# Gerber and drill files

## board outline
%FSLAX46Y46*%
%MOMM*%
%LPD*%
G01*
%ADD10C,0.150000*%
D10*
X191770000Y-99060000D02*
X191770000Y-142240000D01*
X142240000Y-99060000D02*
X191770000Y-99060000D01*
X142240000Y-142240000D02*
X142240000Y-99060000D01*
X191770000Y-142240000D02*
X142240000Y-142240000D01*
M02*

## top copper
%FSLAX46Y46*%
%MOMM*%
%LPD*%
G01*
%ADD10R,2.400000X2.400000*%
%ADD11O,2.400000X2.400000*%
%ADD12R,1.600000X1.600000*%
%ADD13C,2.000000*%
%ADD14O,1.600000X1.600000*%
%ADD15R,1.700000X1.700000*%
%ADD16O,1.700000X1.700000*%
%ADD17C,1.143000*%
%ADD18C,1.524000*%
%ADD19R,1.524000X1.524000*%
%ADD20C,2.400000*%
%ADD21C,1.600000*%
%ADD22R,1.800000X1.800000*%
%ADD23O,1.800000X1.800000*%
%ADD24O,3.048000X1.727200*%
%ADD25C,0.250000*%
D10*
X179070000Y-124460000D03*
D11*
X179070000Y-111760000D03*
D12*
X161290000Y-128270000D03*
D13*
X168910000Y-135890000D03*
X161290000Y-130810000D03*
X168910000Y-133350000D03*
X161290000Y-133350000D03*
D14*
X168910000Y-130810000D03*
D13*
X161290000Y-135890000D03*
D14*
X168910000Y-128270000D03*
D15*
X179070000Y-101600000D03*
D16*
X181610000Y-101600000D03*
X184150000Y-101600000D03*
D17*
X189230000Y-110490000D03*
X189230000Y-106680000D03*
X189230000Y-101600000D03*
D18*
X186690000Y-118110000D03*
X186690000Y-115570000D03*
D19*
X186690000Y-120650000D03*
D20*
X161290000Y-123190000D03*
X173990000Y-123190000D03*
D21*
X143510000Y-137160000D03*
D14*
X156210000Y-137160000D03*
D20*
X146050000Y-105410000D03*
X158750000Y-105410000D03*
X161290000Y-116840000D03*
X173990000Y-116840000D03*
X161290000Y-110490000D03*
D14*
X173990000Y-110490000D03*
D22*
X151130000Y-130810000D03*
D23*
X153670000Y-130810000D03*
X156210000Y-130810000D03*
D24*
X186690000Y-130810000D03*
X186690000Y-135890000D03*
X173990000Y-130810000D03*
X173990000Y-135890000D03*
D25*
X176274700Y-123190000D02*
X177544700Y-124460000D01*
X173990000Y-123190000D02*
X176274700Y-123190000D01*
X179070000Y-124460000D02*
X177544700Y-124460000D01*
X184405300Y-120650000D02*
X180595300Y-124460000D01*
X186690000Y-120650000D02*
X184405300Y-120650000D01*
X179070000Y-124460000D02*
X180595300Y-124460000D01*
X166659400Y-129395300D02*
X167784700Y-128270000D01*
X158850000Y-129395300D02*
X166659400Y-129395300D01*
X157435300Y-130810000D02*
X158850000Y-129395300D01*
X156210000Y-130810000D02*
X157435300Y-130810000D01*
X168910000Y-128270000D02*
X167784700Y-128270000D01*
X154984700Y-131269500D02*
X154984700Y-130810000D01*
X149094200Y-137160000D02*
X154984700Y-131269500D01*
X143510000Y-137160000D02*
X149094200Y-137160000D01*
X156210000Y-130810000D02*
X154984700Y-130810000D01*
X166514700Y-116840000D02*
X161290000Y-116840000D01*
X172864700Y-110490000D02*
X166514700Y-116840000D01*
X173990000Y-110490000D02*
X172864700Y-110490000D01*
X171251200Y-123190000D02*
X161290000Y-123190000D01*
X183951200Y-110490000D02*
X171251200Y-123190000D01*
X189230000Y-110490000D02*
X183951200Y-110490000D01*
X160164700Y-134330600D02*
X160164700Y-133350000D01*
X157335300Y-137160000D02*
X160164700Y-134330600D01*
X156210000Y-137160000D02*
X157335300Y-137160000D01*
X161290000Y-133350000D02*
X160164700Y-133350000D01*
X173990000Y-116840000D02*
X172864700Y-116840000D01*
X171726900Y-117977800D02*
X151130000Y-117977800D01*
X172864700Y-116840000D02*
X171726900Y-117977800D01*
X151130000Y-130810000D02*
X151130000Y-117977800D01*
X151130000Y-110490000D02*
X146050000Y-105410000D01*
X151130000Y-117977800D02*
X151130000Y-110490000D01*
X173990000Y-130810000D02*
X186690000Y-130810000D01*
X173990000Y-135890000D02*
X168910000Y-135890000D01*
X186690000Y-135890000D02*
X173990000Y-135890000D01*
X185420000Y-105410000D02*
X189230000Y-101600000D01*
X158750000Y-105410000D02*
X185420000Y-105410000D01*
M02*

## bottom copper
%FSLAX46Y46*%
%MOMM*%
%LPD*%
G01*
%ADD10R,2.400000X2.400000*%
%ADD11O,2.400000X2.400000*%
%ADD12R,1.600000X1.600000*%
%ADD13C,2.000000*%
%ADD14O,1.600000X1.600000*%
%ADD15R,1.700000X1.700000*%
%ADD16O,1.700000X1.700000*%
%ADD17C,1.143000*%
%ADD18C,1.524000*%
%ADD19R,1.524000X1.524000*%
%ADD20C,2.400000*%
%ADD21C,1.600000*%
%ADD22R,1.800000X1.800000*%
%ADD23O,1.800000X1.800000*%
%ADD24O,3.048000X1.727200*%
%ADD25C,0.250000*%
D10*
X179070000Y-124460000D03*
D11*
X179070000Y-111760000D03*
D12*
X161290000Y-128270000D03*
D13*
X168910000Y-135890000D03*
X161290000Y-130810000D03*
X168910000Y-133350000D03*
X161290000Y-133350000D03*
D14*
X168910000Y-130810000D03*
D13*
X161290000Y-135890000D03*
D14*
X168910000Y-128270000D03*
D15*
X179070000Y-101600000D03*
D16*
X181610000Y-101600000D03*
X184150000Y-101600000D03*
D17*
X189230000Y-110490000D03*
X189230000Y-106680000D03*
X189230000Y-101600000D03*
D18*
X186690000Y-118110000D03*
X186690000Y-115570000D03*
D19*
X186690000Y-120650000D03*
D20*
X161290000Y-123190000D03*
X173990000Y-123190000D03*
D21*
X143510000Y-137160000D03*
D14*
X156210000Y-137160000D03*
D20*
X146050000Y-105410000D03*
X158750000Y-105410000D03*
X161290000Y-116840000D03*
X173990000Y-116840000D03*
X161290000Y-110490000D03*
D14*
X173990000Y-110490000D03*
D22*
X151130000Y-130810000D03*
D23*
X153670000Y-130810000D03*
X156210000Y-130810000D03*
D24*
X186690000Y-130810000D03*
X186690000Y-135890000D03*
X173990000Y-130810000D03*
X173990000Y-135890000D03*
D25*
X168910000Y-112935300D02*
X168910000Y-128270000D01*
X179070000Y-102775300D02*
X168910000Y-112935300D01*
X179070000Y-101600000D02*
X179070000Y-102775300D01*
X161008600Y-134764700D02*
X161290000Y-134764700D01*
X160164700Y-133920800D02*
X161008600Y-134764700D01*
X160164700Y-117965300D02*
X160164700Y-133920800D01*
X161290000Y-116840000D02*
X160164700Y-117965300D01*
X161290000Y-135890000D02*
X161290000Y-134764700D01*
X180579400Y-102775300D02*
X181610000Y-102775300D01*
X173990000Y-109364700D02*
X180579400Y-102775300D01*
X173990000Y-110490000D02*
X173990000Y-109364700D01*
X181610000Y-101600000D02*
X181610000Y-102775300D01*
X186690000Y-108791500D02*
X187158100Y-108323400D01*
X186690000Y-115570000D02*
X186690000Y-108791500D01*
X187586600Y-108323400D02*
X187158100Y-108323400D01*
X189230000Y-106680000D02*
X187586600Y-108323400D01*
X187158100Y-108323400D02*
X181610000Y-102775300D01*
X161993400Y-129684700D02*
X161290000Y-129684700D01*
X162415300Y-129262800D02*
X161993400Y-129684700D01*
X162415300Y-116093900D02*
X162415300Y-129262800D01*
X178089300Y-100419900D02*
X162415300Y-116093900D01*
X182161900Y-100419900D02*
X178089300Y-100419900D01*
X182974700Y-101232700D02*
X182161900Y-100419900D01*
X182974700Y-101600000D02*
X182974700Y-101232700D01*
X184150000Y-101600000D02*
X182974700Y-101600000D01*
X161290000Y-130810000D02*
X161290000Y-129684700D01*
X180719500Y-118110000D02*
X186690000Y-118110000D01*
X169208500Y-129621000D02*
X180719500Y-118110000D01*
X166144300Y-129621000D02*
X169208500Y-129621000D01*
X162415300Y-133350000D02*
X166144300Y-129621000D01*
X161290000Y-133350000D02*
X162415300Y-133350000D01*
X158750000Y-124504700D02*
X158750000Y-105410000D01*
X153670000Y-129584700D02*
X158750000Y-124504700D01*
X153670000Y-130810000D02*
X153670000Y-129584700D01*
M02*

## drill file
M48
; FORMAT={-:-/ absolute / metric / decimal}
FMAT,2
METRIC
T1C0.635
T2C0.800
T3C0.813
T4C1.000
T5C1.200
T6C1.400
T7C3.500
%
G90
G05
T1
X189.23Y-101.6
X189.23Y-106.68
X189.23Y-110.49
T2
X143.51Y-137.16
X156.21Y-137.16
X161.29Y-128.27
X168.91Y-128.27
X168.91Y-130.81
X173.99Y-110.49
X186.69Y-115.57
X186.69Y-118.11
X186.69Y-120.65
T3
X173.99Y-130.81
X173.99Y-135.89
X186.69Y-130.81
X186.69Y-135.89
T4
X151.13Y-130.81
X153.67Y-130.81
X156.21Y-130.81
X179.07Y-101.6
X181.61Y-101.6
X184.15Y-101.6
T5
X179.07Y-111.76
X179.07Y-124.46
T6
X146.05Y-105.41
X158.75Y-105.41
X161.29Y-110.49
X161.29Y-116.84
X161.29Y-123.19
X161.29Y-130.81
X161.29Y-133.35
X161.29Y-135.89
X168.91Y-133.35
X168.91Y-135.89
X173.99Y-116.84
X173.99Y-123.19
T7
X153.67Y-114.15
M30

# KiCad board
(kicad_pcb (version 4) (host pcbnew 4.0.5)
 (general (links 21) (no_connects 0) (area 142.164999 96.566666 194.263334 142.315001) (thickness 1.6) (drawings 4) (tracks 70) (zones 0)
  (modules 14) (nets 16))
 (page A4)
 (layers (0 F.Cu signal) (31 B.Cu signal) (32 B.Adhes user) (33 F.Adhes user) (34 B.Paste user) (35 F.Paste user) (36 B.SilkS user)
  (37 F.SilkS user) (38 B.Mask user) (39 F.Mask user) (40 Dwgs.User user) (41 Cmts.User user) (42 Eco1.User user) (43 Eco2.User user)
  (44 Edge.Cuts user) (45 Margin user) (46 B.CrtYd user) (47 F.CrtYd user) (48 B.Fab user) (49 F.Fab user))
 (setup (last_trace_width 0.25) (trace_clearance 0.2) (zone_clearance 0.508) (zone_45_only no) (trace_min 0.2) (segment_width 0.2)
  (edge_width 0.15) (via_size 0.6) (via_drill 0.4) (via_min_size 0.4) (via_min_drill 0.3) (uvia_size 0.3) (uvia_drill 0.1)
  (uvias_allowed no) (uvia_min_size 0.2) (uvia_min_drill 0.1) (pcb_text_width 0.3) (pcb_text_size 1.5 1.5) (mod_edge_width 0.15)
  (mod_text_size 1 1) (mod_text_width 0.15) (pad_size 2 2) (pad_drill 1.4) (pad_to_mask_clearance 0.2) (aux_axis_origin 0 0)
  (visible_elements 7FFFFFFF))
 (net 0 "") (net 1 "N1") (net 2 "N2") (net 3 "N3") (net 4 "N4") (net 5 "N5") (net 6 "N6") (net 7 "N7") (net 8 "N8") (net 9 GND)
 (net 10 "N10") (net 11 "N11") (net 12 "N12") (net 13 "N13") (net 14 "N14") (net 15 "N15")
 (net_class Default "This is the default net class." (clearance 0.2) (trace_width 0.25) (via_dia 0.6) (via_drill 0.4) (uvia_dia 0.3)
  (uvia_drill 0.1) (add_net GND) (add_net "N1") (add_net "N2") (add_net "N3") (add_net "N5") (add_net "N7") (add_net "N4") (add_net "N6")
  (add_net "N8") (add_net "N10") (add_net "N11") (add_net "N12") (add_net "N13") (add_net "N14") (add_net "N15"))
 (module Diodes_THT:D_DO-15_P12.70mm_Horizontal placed (layer F.Cu) (at 179.07 124.46 90)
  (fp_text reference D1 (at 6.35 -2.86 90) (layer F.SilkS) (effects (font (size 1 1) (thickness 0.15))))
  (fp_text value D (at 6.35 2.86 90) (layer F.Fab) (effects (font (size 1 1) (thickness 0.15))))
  (pad 1 thru_hole rect (at 0 0 90) (size 2.4 2.4) (drill 1.2) (layers *.Cu *.Mask) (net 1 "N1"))
  (pad 2 thru_hole oval (at 12.7 0 90) (size 2.4 2.4) (drill 1.2) (layers *.Cu *.Mask) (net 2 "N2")))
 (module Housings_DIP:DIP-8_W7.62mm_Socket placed (layer F.Cu) (at 161.29 128.27)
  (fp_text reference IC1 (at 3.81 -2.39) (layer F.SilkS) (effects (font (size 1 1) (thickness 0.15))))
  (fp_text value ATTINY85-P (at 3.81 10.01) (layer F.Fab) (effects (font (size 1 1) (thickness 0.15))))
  (pad 1 thru_hole rect (at 0 0) (size 1.6 1.6) (drill 0.8) (layers *.Cu *.Mask) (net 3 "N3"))
  (pad 5 thru_hole circle (at 7.62 7.62) (size 2 2) (drill 1.4) (layers *.Cu *.Mask) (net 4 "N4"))
  (pad 2 thru_hole circle (at 0 2.54) (size 2 2) (drill 1.4) (layers *.Cu *.Mask) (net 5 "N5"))
  (pad 6 thru_hole circle (at 7.62 5.08) (size 2 2) (drill 1.4) (layers *.Cu *.Mask) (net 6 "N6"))
  (pad 3 thru_hole circle (at 0 5.08) (size 2 2) (drill 1.4) (layers *.Cu *.Mask) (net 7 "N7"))
  (pad 7 thru_hole oval (at 7.62 2.54) (size 1.6 1.6) (drill 0.8) (layers *.Cu *.Mask) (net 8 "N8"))
  (pad 4 thru_hole circle (at 0 7.62) (size 2 2) (drill 1.4) (layers *.Cu *.Mask) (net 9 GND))
  (pad 8 thru_hole oval (at 7.62 0) (size 1.6 1.6) (drill 0.8) (layers *.Cu *.Mask) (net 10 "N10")))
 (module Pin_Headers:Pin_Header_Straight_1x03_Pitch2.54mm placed (layer F.Cu) (at 179.07 101.6 90)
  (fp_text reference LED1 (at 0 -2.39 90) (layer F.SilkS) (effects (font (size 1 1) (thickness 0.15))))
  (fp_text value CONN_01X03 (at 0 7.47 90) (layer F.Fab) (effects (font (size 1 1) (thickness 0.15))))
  (pad 1 thru_hole rect (at 0 0 90) (size 1.7 1.7) (drill 1) (layers *.Cu *.Mask) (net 10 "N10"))
  (pad 2 thru_hole oval (at 0 2.54 90) (size 1.7 1.7) (drill 1) (layers *.Cu *.Mask) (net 9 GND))
  (pad 3 thru_hole oval (at 0 5.08 90) (size 1.7 1.7) (drill 1) (layers *.Cu *.Mask) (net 5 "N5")))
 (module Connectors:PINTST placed (layer F.Cu) (at 189.23 110.49)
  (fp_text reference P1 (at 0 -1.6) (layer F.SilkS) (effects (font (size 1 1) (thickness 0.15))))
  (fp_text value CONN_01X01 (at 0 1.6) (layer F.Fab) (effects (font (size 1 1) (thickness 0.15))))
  (pad 1 thru_hole circle (at 0 0) (size 1.143 1.143) (drill 0.635) (layers *.Cu *.Mask) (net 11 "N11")))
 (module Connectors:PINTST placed (layer F.Cu) (at 189.23 106.68)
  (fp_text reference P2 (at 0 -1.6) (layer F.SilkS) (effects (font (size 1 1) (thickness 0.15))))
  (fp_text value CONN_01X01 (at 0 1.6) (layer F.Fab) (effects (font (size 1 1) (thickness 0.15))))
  (pad 1 thru_hole circle (at 0 0) (size 1.143 1.143) (drill 0.635) (layers *.Cu *.Mask) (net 9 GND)))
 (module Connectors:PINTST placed (layer F.Cu) (at 189.23 101.6)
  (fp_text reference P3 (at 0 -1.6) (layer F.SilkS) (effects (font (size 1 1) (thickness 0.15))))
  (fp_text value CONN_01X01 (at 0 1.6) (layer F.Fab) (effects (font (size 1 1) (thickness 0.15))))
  (pad 1 thru_hole circle (at 0 0) (size 1.143 1.143) (drill 0.635) (layers *.Cu *.Mask) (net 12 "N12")))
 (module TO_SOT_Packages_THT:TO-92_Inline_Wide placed (layer F.Cu) (at 186.69 120.65 90)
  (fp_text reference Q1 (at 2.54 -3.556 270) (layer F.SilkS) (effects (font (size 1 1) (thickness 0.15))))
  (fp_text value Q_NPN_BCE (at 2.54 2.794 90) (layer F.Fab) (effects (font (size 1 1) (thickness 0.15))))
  (pad 2 thru_hole circle (at 2.54 0 180) (size 1.524 1.524) (drill 0.8) (layers *.Cu *.Mask) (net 7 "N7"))
  (pad 3 thru_hole circle (at 5.08 0 180) (size 1.524 1.524) (drill 0.8) (layers *.Cu *.Mask) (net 9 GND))
  (pad 1 thru_hole rect (at 0 0 180) (size 1.524 1.524) (drill 0.8) (layers *.Cu *.Mask) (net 1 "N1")))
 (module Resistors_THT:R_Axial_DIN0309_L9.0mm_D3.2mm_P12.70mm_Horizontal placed (layer F.Cu) (at 161.29 123.19)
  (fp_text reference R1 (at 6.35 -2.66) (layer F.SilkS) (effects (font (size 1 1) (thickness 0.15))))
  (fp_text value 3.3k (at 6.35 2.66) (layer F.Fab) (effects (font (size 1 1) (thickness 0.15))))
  (pad 1 thru_hole circle (at 0 0) (size 2.4 2.4) (drill 1.4) (layers *.Cu *.Mask) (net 11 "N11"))
  (pad 2 thru_hole circle (at 12.7 0) (size 2.4 2.4) (drill 1.4) (layers *.Cu *.Mask) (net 1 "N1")))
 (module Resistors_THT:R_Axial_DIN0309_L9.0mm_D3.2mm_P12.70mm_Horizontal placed (layer F.Cu) (at 143.51 137.16)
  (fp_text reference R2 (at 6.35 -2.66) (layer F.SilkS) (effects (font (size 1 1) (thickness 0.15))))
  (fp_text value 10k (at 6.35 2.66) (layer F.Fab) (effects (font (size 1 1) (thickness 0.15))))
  (pad 1 thru_hole circle (at 0 0) (size 1.6 1.6) (drill 0.8) (layers *.Cu *.Mask) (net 10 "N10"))
  (pad 2 thru_hole oval (at 12.7 0) (size 1.6 1.6) (drill 0.8) (layers *.Cu *.Mask) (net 7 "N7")))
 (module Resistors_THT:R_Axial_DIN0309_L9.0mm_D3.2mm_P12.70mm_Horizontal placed (layer F.Cu) (at 146.05 105.41)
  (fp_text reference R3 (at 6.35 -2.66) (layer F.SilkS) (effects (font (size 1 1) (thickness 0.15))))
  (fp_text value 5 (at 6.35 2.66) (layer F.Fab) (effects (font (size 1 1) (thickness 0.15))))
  (pad 1 thru_hole circle (at 0 0) (size 2.4 2.4) (drill 1.4) (layers *.Cu *.Mask) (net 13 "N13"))
  (pad 2 thru_hole circle (at 12.7 0) (size 2.4 2.4) (drill 1.4) (layers *.Cu *.Mask) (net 12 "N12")))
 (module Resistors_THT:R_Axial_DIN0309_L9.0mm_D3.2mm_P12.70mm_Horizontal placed (layer F.Cu) (at 161.29 116.84)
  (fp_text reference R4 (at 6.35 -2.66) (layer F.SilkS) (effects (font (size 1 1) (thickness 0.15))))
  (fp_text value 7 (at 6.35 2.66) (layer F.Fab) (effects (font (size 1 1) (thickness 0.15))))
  (pad 1 thru_hole circle (at 0 0) (size 2.4 2.4) (drill 1.4) (layers *.Cu *.Mask) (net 9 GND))
  (pad 2 thru_hole circle (at 12.7 0) (size 2.4 2.4) (drill 1.4) (layers *.Cu *.Mask) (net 13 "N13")))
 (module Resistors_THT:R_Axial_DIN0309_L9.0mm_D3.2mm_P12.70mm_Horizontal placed (layer F.Cu) (at 161.29 110.49)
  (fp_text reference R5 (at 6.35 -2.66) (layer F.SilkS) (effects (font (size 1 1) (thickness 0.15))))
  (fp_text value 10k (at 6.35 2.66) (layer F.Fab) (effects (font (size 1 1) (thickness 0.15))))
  (pad 1 thru_hole circle (at 0 0) (size 2.4 2.4) (drill 1.4) (layers *.Cu *.Mask) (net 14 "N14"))
  (pad 2 thru_hole oval (at 12.7 0) (size 1.6 1.6) (drill 0.8) (layers *.Cu *.Mask) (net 9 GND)))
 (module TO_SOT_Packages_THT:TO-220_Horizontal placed (layer F.Cu) (at 151.13 130.81)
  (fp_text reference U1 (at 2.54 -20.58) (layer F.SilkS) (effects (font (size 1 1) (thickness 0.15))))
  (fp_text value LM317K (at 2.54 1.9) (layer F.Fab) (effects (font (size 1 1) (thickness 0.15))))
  (pad None np_thru_hole oval (at 2.54 -16.66) (size 3.5 3.5) (drill 3.5) (layers *.Cu *.Mask))
  (pad 1 thru_hole rect (at 0 0) (size 1.8 1.8) (drill 1) (layers *.Cu *.Mask) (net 13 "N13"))
  (pad 2 thru_hole oval (at 2.54 0) (size 1.8 1.8) (drill 1) (layers *.Cu *.Mask) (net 12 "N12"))
  (pad 3 thru_hole oval (at 5.08 0) (size 1.8 1.8) (drill 1) (layers *.Cu *.Mask) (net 10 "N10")))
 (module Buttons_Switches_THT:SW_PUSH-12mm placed (layer F.Cu) (at 180.34 133.35)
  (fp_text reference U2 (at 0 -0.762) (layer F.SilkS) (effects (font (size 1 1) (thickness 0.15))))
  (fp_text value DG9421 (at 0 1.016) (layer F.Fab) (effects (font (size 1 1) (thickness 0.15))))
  (pad 1 thru_hole oval (at 6.35 -2.54) (size 3.048 1.7272) (drill 0.8128) (layers *.Cu *.Mask) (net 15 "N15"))
  (pad 2 thru_hole oval (at 6.35 2.54) (size 3.048 1.7272) (drill 0.8128) (layers *.Cu *.Mask) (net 4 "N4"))
  (pad 1 thru_hole oval (at -6.35 -2.54) (size 3.048 1.7272) (drill 0.8128) (layers *.Cu *.Mask) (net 15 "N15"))
  (pad 2 thru_hole oval (at -6.35 2.54) (size 3.048 1.7272) (drill 0.8128) (layers *.Cu *.Mask) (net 4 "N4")))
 (gr_line (start 191.77 99.06) (end 191.77 142.24) (angle 90) (layer Edge.Cuts) (width 0.15))
 (gr_line (start 142.24 99.06) (end 191.77 99.06) (angle 90) (layer Edge.Cuts) (width 0.15))
 (gr_line (start 142.24 142.24) (end 142.24 99.06) (angle 90) (layer Edge.Cuts) (width 0.15))
 (gr_line (start 191.77 142.24) (end 142.24 142.24) (angle 90) (layer Edge.Cuts) (width 0.15))
 (segment (start 176.2747 123.19) (end 177.5447 124.46) (width 0.25) (layer F.Cu) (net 1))
 (segment (start 173.99 123.19) (end 176.2747 123.19) (width 0.25) (layer F.Cu) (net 1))
 (segment (start 179.07 124.46) (end 177.5447 124.46) (width 0.25) (layer F.Cu) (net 1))
 (segment (start 184.4053 120.65) (end 180.5953 124.46) (width 0.25) (layer F.Cu) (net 1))
 (segment (start 186.69 120.65) (end 184.4053 120.65) (width 0.25) (layer F.Cu) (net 1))
 (segment (start 179.07 124.46) (end 180.5953 124.46) (width 0.25) (layer F.Cu) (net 1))
 (segment (start 166.6594 129.3953) (end 167.7847 128.27) (width 0.25) (layer F.Cu) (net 10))
 (segment (start 158.85 129.3953) (end 166.6594 129.3953) (width 0.25) (layer F.Cu) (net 10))
 (segment (start 157.4353 130.81) (end 158.85 129.3953) (width 0.25) (layer F.Cu) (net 10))
 (segment (start 156.21 130.81) (end 157.4353 130.81) (width 0.25) (layer F.Cu) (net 10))
 (segment (start 168.91 128.27) (end 167.7847 128.27) (width 0.25) (layer F.Cu) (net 10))
 (segment (start 154.9847 131.2695) (end 154.9847 130.81) (width 0.25) (layer F.Cu) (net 10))
 (segment (start 149.0942 137.16) (end 154.9847 131.2695) (width 0.25) (layer F.Cu) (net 10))
 (segment (start 143.51 137.16) (end 149.0942 137.16) (width 0.25) (layer F.Cu) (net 10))
 (segment (start 156.21 130.81) (end 154.9847 130.81) (width 0.25) (layer F.Cu) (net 10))
 (segment (start 168.91 112.9353) (end 168.91 128.27) (width 0.25) (layer B.Cu) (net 10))
 (segment (start 179.07 102.7753) (end 168.91 112.9353) (width 0.25) (layer B.Cu) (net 10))
 (segment (start 179.07 101.6) (end 179.07 102.7753) (width 0.25) (layer B.Cu) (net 10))
 (segment (start 161.0086 134.7647) (end 161.29 134.7647) (width 0.25) (layer B.Cu) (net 9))
 (segment (start 160.1647 133.9208) (end 161.0086 134.7647) (width 0.25) (layer B.Cu) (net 9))
 (segment (start 160.1647 117.9653) (end 160.1647 133.9208) (width 0.25) (layer B.Cu) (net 9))
 (segment (start 161.29 116.84) (end 160.1647 117.9653) (width 0.25) (layer B.Cu) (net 9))
 (segment (start 161.29 135.89) (end 161.29 134.7647) (width 0.25) (layer B.Cu) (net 9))
 (segment (start 166.5147 116.84) (end 161.29 116.84) (width 0.25) (layer F.Cu) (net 9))
 (segment (start 172.8647 110.49) (end 166.5147 116.84) (width 0.25) (layer F.Cu) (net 9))
 (segment (start 173.99 110.49) (end 172.8647 110.49) (width 0.25) (layer F.Cu) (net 9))
 (segment (start 180.5794 102.7753) (end 181.61 102.7753) (width 0.25) (layer B.Cu) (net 9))
 (segment (start 173.99 109.3647) (end 180.5794 102.7753) (width 0.25) (layer B.Cu) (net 9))
 (segment (start 173.99 110.49) (end 173.99 109.3647) (width 0.25) (layer B.Cu) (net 9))
 (segment (start 181.61 101.6) (end 181.61 102.7753) (width 0.25) (layer B.Cu) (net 9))
 (segment (start 186.69 108.7915) (end 187.1581 108.3234) (width 0.25) (layer B.Cu) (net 9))
 (segment (start 186.69 115.57) (end 186.69 108.7915) (width 0.25) (layer B.Cu) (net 9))
 (segment (start 187.5866 108.3234) (end 187.1581 108.3234) (width 0.25) (layer B.Cu) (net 9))
 (segment (start 189.23 106.68) (end 187.5866 108.3234) (width 0.25) (layer B.Cu) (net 9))
 (segment (start 187.1581 108.3234) (end 181.61 102.7753) (width 0.25) (layer B.Cu) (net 9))
 (segment (start 161.9934 129.6847) (end 161.29 129.6847) (width 0.25) (layer B.Cu) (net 5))
 (segment (start 162.4153 129.2628) (end 161.9934 129.6847) (width 0.25) (layer B.Cu) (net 5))
 (segment (start 162.4153 116.0939) (end 162.4153 129.2628) (width 0.25) (layer B.Cu) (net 5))
 (segment (start 178.0893 100.4199) (end 162.4153 116.0939) (width 0.25) (layer B.Cu) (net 5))
 (segment (start 182.1619 100.4199) (end 178.0893 100.4199) (width 0.25) (layer B.Cu) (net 5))
 (segment (start 182.9747 101.2327) (end 182.1619 100.4199) (width 0.25) (layer B.Cu) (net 5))
 (segment (start 182.9747 101.6) (end 182.9747 101.2327) (width 0.25) (layer B.Cu) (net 5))
 (segment (start 184.15 101.6) (end 182.9747 101.6) (width 0.25) (layer B.Cu) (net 5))
 (segment (start 161.29 130.81) (end 161.29 129.6847) (width 0.25) (layer B.Cu) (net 5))
 (segment (start 171.2512 123.19) (end 161.29 123.19) (width 0.25) (layer F.Cu) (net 11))
 (segment (start 183.9512 110.49) (end 171.2512 123.19) (width 0.25) (layer F.Cu) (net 11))
 (segment (start 189.23 110.49) (end 183.9512 110.49) (width 0.25) (layer F.Cu) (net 11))
 (segment (start 180.7195 118.11) (end 186.69 118.11) (width 0.25) (layer B.Cu) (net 7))
 (segment (start 169.2085 129.621) (end 180.7195 118.11) (width 0.25) (layer B.Cu) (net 7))
 (segment (start 166.1443 129.621) (end 169.2085 129.621) (width 0.25) (layer B.Cu) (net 7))
 (segment (start 162.4153 133.35) (end 166.1443 129.621) (width 0.25) (layer B.Cu) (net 7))
 (segment (start 161.29 133.35) (end 162.4153 133.35) (width 0.25) (layer B.Cu) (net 7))
 (segment (start 160.1647 134.3306) (end 160.1647 133.35) (width 0.25) (layer F.Cu) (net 7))
 (segment (start 157.3353 137.16) (end 160.1647 134.3306) (width 0.25) (layer F.Cu) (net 7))
 (segment (start 156.21 137.16) (end 157.3353 137.16) (width 0.25) (layer F.Cu) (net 7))
 (segment (start 161.29 133.35) (end 160.1647 133.35) (width 0.25) (layer F.Cu) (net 7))
 (segment (start 173.99 116.84) (end 172.8647 116.84) (width 0.25) (layer F.Cu) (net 13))
 (segment (start 171.7269 117.9778) (end 151.13 117.9778) (width 0.25) (layer F.Cu) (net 13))
 (segment (start 172.8647 116.84) (end 171.7269 117.9778) (width 0.25) (layer F.Cu) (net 13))
 (segment (start 151.13 130.81) (end 151.13 117.9778) (width 0.25) (layer F.Cu) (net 13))
 (segment (start 151.13 110.49) (end 146.05 105.41) (width 0.25) (layer F.Cu) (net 13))
 (segment (start 151.13 117.9778) (end 151.13 110.49) (width 0.25) (layer F.Cu) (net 13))
 (segment (start 173.99 130.81) (end 186.69 130.81) (width 0.25) (layer F.Cu) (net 15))
 (segment (start 173.99 135.89) (end 168.91 135.89) (width 0.25) (layer F.Cu) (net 4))
 (segment (start 186.69 135.89) (end 173.99 135.89) (width 0.25) (layer F.Cu) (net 4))
 (segment (start 158.75 124.5047) (end 158.75 105.41) (width 0.25) (layer B.Cu) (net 12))
 (segment (start 153.67 129.5847) (end 158.75 124.5047) (width 0.25) (layer B.Cu) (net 12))
 (segment (start 153.67 130.81) (end 153.67 129.5847) (width 0.25) (layer B.Cu) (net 12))
 (segment (start 185.42 105.41) (end 189.23 101.6) (width 0.25) (layer F.Cu) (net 12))
 (segment (start 158.75 105.41) (end 185.42 105.41) (width 0.25) (layer F.Cu) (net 12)))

